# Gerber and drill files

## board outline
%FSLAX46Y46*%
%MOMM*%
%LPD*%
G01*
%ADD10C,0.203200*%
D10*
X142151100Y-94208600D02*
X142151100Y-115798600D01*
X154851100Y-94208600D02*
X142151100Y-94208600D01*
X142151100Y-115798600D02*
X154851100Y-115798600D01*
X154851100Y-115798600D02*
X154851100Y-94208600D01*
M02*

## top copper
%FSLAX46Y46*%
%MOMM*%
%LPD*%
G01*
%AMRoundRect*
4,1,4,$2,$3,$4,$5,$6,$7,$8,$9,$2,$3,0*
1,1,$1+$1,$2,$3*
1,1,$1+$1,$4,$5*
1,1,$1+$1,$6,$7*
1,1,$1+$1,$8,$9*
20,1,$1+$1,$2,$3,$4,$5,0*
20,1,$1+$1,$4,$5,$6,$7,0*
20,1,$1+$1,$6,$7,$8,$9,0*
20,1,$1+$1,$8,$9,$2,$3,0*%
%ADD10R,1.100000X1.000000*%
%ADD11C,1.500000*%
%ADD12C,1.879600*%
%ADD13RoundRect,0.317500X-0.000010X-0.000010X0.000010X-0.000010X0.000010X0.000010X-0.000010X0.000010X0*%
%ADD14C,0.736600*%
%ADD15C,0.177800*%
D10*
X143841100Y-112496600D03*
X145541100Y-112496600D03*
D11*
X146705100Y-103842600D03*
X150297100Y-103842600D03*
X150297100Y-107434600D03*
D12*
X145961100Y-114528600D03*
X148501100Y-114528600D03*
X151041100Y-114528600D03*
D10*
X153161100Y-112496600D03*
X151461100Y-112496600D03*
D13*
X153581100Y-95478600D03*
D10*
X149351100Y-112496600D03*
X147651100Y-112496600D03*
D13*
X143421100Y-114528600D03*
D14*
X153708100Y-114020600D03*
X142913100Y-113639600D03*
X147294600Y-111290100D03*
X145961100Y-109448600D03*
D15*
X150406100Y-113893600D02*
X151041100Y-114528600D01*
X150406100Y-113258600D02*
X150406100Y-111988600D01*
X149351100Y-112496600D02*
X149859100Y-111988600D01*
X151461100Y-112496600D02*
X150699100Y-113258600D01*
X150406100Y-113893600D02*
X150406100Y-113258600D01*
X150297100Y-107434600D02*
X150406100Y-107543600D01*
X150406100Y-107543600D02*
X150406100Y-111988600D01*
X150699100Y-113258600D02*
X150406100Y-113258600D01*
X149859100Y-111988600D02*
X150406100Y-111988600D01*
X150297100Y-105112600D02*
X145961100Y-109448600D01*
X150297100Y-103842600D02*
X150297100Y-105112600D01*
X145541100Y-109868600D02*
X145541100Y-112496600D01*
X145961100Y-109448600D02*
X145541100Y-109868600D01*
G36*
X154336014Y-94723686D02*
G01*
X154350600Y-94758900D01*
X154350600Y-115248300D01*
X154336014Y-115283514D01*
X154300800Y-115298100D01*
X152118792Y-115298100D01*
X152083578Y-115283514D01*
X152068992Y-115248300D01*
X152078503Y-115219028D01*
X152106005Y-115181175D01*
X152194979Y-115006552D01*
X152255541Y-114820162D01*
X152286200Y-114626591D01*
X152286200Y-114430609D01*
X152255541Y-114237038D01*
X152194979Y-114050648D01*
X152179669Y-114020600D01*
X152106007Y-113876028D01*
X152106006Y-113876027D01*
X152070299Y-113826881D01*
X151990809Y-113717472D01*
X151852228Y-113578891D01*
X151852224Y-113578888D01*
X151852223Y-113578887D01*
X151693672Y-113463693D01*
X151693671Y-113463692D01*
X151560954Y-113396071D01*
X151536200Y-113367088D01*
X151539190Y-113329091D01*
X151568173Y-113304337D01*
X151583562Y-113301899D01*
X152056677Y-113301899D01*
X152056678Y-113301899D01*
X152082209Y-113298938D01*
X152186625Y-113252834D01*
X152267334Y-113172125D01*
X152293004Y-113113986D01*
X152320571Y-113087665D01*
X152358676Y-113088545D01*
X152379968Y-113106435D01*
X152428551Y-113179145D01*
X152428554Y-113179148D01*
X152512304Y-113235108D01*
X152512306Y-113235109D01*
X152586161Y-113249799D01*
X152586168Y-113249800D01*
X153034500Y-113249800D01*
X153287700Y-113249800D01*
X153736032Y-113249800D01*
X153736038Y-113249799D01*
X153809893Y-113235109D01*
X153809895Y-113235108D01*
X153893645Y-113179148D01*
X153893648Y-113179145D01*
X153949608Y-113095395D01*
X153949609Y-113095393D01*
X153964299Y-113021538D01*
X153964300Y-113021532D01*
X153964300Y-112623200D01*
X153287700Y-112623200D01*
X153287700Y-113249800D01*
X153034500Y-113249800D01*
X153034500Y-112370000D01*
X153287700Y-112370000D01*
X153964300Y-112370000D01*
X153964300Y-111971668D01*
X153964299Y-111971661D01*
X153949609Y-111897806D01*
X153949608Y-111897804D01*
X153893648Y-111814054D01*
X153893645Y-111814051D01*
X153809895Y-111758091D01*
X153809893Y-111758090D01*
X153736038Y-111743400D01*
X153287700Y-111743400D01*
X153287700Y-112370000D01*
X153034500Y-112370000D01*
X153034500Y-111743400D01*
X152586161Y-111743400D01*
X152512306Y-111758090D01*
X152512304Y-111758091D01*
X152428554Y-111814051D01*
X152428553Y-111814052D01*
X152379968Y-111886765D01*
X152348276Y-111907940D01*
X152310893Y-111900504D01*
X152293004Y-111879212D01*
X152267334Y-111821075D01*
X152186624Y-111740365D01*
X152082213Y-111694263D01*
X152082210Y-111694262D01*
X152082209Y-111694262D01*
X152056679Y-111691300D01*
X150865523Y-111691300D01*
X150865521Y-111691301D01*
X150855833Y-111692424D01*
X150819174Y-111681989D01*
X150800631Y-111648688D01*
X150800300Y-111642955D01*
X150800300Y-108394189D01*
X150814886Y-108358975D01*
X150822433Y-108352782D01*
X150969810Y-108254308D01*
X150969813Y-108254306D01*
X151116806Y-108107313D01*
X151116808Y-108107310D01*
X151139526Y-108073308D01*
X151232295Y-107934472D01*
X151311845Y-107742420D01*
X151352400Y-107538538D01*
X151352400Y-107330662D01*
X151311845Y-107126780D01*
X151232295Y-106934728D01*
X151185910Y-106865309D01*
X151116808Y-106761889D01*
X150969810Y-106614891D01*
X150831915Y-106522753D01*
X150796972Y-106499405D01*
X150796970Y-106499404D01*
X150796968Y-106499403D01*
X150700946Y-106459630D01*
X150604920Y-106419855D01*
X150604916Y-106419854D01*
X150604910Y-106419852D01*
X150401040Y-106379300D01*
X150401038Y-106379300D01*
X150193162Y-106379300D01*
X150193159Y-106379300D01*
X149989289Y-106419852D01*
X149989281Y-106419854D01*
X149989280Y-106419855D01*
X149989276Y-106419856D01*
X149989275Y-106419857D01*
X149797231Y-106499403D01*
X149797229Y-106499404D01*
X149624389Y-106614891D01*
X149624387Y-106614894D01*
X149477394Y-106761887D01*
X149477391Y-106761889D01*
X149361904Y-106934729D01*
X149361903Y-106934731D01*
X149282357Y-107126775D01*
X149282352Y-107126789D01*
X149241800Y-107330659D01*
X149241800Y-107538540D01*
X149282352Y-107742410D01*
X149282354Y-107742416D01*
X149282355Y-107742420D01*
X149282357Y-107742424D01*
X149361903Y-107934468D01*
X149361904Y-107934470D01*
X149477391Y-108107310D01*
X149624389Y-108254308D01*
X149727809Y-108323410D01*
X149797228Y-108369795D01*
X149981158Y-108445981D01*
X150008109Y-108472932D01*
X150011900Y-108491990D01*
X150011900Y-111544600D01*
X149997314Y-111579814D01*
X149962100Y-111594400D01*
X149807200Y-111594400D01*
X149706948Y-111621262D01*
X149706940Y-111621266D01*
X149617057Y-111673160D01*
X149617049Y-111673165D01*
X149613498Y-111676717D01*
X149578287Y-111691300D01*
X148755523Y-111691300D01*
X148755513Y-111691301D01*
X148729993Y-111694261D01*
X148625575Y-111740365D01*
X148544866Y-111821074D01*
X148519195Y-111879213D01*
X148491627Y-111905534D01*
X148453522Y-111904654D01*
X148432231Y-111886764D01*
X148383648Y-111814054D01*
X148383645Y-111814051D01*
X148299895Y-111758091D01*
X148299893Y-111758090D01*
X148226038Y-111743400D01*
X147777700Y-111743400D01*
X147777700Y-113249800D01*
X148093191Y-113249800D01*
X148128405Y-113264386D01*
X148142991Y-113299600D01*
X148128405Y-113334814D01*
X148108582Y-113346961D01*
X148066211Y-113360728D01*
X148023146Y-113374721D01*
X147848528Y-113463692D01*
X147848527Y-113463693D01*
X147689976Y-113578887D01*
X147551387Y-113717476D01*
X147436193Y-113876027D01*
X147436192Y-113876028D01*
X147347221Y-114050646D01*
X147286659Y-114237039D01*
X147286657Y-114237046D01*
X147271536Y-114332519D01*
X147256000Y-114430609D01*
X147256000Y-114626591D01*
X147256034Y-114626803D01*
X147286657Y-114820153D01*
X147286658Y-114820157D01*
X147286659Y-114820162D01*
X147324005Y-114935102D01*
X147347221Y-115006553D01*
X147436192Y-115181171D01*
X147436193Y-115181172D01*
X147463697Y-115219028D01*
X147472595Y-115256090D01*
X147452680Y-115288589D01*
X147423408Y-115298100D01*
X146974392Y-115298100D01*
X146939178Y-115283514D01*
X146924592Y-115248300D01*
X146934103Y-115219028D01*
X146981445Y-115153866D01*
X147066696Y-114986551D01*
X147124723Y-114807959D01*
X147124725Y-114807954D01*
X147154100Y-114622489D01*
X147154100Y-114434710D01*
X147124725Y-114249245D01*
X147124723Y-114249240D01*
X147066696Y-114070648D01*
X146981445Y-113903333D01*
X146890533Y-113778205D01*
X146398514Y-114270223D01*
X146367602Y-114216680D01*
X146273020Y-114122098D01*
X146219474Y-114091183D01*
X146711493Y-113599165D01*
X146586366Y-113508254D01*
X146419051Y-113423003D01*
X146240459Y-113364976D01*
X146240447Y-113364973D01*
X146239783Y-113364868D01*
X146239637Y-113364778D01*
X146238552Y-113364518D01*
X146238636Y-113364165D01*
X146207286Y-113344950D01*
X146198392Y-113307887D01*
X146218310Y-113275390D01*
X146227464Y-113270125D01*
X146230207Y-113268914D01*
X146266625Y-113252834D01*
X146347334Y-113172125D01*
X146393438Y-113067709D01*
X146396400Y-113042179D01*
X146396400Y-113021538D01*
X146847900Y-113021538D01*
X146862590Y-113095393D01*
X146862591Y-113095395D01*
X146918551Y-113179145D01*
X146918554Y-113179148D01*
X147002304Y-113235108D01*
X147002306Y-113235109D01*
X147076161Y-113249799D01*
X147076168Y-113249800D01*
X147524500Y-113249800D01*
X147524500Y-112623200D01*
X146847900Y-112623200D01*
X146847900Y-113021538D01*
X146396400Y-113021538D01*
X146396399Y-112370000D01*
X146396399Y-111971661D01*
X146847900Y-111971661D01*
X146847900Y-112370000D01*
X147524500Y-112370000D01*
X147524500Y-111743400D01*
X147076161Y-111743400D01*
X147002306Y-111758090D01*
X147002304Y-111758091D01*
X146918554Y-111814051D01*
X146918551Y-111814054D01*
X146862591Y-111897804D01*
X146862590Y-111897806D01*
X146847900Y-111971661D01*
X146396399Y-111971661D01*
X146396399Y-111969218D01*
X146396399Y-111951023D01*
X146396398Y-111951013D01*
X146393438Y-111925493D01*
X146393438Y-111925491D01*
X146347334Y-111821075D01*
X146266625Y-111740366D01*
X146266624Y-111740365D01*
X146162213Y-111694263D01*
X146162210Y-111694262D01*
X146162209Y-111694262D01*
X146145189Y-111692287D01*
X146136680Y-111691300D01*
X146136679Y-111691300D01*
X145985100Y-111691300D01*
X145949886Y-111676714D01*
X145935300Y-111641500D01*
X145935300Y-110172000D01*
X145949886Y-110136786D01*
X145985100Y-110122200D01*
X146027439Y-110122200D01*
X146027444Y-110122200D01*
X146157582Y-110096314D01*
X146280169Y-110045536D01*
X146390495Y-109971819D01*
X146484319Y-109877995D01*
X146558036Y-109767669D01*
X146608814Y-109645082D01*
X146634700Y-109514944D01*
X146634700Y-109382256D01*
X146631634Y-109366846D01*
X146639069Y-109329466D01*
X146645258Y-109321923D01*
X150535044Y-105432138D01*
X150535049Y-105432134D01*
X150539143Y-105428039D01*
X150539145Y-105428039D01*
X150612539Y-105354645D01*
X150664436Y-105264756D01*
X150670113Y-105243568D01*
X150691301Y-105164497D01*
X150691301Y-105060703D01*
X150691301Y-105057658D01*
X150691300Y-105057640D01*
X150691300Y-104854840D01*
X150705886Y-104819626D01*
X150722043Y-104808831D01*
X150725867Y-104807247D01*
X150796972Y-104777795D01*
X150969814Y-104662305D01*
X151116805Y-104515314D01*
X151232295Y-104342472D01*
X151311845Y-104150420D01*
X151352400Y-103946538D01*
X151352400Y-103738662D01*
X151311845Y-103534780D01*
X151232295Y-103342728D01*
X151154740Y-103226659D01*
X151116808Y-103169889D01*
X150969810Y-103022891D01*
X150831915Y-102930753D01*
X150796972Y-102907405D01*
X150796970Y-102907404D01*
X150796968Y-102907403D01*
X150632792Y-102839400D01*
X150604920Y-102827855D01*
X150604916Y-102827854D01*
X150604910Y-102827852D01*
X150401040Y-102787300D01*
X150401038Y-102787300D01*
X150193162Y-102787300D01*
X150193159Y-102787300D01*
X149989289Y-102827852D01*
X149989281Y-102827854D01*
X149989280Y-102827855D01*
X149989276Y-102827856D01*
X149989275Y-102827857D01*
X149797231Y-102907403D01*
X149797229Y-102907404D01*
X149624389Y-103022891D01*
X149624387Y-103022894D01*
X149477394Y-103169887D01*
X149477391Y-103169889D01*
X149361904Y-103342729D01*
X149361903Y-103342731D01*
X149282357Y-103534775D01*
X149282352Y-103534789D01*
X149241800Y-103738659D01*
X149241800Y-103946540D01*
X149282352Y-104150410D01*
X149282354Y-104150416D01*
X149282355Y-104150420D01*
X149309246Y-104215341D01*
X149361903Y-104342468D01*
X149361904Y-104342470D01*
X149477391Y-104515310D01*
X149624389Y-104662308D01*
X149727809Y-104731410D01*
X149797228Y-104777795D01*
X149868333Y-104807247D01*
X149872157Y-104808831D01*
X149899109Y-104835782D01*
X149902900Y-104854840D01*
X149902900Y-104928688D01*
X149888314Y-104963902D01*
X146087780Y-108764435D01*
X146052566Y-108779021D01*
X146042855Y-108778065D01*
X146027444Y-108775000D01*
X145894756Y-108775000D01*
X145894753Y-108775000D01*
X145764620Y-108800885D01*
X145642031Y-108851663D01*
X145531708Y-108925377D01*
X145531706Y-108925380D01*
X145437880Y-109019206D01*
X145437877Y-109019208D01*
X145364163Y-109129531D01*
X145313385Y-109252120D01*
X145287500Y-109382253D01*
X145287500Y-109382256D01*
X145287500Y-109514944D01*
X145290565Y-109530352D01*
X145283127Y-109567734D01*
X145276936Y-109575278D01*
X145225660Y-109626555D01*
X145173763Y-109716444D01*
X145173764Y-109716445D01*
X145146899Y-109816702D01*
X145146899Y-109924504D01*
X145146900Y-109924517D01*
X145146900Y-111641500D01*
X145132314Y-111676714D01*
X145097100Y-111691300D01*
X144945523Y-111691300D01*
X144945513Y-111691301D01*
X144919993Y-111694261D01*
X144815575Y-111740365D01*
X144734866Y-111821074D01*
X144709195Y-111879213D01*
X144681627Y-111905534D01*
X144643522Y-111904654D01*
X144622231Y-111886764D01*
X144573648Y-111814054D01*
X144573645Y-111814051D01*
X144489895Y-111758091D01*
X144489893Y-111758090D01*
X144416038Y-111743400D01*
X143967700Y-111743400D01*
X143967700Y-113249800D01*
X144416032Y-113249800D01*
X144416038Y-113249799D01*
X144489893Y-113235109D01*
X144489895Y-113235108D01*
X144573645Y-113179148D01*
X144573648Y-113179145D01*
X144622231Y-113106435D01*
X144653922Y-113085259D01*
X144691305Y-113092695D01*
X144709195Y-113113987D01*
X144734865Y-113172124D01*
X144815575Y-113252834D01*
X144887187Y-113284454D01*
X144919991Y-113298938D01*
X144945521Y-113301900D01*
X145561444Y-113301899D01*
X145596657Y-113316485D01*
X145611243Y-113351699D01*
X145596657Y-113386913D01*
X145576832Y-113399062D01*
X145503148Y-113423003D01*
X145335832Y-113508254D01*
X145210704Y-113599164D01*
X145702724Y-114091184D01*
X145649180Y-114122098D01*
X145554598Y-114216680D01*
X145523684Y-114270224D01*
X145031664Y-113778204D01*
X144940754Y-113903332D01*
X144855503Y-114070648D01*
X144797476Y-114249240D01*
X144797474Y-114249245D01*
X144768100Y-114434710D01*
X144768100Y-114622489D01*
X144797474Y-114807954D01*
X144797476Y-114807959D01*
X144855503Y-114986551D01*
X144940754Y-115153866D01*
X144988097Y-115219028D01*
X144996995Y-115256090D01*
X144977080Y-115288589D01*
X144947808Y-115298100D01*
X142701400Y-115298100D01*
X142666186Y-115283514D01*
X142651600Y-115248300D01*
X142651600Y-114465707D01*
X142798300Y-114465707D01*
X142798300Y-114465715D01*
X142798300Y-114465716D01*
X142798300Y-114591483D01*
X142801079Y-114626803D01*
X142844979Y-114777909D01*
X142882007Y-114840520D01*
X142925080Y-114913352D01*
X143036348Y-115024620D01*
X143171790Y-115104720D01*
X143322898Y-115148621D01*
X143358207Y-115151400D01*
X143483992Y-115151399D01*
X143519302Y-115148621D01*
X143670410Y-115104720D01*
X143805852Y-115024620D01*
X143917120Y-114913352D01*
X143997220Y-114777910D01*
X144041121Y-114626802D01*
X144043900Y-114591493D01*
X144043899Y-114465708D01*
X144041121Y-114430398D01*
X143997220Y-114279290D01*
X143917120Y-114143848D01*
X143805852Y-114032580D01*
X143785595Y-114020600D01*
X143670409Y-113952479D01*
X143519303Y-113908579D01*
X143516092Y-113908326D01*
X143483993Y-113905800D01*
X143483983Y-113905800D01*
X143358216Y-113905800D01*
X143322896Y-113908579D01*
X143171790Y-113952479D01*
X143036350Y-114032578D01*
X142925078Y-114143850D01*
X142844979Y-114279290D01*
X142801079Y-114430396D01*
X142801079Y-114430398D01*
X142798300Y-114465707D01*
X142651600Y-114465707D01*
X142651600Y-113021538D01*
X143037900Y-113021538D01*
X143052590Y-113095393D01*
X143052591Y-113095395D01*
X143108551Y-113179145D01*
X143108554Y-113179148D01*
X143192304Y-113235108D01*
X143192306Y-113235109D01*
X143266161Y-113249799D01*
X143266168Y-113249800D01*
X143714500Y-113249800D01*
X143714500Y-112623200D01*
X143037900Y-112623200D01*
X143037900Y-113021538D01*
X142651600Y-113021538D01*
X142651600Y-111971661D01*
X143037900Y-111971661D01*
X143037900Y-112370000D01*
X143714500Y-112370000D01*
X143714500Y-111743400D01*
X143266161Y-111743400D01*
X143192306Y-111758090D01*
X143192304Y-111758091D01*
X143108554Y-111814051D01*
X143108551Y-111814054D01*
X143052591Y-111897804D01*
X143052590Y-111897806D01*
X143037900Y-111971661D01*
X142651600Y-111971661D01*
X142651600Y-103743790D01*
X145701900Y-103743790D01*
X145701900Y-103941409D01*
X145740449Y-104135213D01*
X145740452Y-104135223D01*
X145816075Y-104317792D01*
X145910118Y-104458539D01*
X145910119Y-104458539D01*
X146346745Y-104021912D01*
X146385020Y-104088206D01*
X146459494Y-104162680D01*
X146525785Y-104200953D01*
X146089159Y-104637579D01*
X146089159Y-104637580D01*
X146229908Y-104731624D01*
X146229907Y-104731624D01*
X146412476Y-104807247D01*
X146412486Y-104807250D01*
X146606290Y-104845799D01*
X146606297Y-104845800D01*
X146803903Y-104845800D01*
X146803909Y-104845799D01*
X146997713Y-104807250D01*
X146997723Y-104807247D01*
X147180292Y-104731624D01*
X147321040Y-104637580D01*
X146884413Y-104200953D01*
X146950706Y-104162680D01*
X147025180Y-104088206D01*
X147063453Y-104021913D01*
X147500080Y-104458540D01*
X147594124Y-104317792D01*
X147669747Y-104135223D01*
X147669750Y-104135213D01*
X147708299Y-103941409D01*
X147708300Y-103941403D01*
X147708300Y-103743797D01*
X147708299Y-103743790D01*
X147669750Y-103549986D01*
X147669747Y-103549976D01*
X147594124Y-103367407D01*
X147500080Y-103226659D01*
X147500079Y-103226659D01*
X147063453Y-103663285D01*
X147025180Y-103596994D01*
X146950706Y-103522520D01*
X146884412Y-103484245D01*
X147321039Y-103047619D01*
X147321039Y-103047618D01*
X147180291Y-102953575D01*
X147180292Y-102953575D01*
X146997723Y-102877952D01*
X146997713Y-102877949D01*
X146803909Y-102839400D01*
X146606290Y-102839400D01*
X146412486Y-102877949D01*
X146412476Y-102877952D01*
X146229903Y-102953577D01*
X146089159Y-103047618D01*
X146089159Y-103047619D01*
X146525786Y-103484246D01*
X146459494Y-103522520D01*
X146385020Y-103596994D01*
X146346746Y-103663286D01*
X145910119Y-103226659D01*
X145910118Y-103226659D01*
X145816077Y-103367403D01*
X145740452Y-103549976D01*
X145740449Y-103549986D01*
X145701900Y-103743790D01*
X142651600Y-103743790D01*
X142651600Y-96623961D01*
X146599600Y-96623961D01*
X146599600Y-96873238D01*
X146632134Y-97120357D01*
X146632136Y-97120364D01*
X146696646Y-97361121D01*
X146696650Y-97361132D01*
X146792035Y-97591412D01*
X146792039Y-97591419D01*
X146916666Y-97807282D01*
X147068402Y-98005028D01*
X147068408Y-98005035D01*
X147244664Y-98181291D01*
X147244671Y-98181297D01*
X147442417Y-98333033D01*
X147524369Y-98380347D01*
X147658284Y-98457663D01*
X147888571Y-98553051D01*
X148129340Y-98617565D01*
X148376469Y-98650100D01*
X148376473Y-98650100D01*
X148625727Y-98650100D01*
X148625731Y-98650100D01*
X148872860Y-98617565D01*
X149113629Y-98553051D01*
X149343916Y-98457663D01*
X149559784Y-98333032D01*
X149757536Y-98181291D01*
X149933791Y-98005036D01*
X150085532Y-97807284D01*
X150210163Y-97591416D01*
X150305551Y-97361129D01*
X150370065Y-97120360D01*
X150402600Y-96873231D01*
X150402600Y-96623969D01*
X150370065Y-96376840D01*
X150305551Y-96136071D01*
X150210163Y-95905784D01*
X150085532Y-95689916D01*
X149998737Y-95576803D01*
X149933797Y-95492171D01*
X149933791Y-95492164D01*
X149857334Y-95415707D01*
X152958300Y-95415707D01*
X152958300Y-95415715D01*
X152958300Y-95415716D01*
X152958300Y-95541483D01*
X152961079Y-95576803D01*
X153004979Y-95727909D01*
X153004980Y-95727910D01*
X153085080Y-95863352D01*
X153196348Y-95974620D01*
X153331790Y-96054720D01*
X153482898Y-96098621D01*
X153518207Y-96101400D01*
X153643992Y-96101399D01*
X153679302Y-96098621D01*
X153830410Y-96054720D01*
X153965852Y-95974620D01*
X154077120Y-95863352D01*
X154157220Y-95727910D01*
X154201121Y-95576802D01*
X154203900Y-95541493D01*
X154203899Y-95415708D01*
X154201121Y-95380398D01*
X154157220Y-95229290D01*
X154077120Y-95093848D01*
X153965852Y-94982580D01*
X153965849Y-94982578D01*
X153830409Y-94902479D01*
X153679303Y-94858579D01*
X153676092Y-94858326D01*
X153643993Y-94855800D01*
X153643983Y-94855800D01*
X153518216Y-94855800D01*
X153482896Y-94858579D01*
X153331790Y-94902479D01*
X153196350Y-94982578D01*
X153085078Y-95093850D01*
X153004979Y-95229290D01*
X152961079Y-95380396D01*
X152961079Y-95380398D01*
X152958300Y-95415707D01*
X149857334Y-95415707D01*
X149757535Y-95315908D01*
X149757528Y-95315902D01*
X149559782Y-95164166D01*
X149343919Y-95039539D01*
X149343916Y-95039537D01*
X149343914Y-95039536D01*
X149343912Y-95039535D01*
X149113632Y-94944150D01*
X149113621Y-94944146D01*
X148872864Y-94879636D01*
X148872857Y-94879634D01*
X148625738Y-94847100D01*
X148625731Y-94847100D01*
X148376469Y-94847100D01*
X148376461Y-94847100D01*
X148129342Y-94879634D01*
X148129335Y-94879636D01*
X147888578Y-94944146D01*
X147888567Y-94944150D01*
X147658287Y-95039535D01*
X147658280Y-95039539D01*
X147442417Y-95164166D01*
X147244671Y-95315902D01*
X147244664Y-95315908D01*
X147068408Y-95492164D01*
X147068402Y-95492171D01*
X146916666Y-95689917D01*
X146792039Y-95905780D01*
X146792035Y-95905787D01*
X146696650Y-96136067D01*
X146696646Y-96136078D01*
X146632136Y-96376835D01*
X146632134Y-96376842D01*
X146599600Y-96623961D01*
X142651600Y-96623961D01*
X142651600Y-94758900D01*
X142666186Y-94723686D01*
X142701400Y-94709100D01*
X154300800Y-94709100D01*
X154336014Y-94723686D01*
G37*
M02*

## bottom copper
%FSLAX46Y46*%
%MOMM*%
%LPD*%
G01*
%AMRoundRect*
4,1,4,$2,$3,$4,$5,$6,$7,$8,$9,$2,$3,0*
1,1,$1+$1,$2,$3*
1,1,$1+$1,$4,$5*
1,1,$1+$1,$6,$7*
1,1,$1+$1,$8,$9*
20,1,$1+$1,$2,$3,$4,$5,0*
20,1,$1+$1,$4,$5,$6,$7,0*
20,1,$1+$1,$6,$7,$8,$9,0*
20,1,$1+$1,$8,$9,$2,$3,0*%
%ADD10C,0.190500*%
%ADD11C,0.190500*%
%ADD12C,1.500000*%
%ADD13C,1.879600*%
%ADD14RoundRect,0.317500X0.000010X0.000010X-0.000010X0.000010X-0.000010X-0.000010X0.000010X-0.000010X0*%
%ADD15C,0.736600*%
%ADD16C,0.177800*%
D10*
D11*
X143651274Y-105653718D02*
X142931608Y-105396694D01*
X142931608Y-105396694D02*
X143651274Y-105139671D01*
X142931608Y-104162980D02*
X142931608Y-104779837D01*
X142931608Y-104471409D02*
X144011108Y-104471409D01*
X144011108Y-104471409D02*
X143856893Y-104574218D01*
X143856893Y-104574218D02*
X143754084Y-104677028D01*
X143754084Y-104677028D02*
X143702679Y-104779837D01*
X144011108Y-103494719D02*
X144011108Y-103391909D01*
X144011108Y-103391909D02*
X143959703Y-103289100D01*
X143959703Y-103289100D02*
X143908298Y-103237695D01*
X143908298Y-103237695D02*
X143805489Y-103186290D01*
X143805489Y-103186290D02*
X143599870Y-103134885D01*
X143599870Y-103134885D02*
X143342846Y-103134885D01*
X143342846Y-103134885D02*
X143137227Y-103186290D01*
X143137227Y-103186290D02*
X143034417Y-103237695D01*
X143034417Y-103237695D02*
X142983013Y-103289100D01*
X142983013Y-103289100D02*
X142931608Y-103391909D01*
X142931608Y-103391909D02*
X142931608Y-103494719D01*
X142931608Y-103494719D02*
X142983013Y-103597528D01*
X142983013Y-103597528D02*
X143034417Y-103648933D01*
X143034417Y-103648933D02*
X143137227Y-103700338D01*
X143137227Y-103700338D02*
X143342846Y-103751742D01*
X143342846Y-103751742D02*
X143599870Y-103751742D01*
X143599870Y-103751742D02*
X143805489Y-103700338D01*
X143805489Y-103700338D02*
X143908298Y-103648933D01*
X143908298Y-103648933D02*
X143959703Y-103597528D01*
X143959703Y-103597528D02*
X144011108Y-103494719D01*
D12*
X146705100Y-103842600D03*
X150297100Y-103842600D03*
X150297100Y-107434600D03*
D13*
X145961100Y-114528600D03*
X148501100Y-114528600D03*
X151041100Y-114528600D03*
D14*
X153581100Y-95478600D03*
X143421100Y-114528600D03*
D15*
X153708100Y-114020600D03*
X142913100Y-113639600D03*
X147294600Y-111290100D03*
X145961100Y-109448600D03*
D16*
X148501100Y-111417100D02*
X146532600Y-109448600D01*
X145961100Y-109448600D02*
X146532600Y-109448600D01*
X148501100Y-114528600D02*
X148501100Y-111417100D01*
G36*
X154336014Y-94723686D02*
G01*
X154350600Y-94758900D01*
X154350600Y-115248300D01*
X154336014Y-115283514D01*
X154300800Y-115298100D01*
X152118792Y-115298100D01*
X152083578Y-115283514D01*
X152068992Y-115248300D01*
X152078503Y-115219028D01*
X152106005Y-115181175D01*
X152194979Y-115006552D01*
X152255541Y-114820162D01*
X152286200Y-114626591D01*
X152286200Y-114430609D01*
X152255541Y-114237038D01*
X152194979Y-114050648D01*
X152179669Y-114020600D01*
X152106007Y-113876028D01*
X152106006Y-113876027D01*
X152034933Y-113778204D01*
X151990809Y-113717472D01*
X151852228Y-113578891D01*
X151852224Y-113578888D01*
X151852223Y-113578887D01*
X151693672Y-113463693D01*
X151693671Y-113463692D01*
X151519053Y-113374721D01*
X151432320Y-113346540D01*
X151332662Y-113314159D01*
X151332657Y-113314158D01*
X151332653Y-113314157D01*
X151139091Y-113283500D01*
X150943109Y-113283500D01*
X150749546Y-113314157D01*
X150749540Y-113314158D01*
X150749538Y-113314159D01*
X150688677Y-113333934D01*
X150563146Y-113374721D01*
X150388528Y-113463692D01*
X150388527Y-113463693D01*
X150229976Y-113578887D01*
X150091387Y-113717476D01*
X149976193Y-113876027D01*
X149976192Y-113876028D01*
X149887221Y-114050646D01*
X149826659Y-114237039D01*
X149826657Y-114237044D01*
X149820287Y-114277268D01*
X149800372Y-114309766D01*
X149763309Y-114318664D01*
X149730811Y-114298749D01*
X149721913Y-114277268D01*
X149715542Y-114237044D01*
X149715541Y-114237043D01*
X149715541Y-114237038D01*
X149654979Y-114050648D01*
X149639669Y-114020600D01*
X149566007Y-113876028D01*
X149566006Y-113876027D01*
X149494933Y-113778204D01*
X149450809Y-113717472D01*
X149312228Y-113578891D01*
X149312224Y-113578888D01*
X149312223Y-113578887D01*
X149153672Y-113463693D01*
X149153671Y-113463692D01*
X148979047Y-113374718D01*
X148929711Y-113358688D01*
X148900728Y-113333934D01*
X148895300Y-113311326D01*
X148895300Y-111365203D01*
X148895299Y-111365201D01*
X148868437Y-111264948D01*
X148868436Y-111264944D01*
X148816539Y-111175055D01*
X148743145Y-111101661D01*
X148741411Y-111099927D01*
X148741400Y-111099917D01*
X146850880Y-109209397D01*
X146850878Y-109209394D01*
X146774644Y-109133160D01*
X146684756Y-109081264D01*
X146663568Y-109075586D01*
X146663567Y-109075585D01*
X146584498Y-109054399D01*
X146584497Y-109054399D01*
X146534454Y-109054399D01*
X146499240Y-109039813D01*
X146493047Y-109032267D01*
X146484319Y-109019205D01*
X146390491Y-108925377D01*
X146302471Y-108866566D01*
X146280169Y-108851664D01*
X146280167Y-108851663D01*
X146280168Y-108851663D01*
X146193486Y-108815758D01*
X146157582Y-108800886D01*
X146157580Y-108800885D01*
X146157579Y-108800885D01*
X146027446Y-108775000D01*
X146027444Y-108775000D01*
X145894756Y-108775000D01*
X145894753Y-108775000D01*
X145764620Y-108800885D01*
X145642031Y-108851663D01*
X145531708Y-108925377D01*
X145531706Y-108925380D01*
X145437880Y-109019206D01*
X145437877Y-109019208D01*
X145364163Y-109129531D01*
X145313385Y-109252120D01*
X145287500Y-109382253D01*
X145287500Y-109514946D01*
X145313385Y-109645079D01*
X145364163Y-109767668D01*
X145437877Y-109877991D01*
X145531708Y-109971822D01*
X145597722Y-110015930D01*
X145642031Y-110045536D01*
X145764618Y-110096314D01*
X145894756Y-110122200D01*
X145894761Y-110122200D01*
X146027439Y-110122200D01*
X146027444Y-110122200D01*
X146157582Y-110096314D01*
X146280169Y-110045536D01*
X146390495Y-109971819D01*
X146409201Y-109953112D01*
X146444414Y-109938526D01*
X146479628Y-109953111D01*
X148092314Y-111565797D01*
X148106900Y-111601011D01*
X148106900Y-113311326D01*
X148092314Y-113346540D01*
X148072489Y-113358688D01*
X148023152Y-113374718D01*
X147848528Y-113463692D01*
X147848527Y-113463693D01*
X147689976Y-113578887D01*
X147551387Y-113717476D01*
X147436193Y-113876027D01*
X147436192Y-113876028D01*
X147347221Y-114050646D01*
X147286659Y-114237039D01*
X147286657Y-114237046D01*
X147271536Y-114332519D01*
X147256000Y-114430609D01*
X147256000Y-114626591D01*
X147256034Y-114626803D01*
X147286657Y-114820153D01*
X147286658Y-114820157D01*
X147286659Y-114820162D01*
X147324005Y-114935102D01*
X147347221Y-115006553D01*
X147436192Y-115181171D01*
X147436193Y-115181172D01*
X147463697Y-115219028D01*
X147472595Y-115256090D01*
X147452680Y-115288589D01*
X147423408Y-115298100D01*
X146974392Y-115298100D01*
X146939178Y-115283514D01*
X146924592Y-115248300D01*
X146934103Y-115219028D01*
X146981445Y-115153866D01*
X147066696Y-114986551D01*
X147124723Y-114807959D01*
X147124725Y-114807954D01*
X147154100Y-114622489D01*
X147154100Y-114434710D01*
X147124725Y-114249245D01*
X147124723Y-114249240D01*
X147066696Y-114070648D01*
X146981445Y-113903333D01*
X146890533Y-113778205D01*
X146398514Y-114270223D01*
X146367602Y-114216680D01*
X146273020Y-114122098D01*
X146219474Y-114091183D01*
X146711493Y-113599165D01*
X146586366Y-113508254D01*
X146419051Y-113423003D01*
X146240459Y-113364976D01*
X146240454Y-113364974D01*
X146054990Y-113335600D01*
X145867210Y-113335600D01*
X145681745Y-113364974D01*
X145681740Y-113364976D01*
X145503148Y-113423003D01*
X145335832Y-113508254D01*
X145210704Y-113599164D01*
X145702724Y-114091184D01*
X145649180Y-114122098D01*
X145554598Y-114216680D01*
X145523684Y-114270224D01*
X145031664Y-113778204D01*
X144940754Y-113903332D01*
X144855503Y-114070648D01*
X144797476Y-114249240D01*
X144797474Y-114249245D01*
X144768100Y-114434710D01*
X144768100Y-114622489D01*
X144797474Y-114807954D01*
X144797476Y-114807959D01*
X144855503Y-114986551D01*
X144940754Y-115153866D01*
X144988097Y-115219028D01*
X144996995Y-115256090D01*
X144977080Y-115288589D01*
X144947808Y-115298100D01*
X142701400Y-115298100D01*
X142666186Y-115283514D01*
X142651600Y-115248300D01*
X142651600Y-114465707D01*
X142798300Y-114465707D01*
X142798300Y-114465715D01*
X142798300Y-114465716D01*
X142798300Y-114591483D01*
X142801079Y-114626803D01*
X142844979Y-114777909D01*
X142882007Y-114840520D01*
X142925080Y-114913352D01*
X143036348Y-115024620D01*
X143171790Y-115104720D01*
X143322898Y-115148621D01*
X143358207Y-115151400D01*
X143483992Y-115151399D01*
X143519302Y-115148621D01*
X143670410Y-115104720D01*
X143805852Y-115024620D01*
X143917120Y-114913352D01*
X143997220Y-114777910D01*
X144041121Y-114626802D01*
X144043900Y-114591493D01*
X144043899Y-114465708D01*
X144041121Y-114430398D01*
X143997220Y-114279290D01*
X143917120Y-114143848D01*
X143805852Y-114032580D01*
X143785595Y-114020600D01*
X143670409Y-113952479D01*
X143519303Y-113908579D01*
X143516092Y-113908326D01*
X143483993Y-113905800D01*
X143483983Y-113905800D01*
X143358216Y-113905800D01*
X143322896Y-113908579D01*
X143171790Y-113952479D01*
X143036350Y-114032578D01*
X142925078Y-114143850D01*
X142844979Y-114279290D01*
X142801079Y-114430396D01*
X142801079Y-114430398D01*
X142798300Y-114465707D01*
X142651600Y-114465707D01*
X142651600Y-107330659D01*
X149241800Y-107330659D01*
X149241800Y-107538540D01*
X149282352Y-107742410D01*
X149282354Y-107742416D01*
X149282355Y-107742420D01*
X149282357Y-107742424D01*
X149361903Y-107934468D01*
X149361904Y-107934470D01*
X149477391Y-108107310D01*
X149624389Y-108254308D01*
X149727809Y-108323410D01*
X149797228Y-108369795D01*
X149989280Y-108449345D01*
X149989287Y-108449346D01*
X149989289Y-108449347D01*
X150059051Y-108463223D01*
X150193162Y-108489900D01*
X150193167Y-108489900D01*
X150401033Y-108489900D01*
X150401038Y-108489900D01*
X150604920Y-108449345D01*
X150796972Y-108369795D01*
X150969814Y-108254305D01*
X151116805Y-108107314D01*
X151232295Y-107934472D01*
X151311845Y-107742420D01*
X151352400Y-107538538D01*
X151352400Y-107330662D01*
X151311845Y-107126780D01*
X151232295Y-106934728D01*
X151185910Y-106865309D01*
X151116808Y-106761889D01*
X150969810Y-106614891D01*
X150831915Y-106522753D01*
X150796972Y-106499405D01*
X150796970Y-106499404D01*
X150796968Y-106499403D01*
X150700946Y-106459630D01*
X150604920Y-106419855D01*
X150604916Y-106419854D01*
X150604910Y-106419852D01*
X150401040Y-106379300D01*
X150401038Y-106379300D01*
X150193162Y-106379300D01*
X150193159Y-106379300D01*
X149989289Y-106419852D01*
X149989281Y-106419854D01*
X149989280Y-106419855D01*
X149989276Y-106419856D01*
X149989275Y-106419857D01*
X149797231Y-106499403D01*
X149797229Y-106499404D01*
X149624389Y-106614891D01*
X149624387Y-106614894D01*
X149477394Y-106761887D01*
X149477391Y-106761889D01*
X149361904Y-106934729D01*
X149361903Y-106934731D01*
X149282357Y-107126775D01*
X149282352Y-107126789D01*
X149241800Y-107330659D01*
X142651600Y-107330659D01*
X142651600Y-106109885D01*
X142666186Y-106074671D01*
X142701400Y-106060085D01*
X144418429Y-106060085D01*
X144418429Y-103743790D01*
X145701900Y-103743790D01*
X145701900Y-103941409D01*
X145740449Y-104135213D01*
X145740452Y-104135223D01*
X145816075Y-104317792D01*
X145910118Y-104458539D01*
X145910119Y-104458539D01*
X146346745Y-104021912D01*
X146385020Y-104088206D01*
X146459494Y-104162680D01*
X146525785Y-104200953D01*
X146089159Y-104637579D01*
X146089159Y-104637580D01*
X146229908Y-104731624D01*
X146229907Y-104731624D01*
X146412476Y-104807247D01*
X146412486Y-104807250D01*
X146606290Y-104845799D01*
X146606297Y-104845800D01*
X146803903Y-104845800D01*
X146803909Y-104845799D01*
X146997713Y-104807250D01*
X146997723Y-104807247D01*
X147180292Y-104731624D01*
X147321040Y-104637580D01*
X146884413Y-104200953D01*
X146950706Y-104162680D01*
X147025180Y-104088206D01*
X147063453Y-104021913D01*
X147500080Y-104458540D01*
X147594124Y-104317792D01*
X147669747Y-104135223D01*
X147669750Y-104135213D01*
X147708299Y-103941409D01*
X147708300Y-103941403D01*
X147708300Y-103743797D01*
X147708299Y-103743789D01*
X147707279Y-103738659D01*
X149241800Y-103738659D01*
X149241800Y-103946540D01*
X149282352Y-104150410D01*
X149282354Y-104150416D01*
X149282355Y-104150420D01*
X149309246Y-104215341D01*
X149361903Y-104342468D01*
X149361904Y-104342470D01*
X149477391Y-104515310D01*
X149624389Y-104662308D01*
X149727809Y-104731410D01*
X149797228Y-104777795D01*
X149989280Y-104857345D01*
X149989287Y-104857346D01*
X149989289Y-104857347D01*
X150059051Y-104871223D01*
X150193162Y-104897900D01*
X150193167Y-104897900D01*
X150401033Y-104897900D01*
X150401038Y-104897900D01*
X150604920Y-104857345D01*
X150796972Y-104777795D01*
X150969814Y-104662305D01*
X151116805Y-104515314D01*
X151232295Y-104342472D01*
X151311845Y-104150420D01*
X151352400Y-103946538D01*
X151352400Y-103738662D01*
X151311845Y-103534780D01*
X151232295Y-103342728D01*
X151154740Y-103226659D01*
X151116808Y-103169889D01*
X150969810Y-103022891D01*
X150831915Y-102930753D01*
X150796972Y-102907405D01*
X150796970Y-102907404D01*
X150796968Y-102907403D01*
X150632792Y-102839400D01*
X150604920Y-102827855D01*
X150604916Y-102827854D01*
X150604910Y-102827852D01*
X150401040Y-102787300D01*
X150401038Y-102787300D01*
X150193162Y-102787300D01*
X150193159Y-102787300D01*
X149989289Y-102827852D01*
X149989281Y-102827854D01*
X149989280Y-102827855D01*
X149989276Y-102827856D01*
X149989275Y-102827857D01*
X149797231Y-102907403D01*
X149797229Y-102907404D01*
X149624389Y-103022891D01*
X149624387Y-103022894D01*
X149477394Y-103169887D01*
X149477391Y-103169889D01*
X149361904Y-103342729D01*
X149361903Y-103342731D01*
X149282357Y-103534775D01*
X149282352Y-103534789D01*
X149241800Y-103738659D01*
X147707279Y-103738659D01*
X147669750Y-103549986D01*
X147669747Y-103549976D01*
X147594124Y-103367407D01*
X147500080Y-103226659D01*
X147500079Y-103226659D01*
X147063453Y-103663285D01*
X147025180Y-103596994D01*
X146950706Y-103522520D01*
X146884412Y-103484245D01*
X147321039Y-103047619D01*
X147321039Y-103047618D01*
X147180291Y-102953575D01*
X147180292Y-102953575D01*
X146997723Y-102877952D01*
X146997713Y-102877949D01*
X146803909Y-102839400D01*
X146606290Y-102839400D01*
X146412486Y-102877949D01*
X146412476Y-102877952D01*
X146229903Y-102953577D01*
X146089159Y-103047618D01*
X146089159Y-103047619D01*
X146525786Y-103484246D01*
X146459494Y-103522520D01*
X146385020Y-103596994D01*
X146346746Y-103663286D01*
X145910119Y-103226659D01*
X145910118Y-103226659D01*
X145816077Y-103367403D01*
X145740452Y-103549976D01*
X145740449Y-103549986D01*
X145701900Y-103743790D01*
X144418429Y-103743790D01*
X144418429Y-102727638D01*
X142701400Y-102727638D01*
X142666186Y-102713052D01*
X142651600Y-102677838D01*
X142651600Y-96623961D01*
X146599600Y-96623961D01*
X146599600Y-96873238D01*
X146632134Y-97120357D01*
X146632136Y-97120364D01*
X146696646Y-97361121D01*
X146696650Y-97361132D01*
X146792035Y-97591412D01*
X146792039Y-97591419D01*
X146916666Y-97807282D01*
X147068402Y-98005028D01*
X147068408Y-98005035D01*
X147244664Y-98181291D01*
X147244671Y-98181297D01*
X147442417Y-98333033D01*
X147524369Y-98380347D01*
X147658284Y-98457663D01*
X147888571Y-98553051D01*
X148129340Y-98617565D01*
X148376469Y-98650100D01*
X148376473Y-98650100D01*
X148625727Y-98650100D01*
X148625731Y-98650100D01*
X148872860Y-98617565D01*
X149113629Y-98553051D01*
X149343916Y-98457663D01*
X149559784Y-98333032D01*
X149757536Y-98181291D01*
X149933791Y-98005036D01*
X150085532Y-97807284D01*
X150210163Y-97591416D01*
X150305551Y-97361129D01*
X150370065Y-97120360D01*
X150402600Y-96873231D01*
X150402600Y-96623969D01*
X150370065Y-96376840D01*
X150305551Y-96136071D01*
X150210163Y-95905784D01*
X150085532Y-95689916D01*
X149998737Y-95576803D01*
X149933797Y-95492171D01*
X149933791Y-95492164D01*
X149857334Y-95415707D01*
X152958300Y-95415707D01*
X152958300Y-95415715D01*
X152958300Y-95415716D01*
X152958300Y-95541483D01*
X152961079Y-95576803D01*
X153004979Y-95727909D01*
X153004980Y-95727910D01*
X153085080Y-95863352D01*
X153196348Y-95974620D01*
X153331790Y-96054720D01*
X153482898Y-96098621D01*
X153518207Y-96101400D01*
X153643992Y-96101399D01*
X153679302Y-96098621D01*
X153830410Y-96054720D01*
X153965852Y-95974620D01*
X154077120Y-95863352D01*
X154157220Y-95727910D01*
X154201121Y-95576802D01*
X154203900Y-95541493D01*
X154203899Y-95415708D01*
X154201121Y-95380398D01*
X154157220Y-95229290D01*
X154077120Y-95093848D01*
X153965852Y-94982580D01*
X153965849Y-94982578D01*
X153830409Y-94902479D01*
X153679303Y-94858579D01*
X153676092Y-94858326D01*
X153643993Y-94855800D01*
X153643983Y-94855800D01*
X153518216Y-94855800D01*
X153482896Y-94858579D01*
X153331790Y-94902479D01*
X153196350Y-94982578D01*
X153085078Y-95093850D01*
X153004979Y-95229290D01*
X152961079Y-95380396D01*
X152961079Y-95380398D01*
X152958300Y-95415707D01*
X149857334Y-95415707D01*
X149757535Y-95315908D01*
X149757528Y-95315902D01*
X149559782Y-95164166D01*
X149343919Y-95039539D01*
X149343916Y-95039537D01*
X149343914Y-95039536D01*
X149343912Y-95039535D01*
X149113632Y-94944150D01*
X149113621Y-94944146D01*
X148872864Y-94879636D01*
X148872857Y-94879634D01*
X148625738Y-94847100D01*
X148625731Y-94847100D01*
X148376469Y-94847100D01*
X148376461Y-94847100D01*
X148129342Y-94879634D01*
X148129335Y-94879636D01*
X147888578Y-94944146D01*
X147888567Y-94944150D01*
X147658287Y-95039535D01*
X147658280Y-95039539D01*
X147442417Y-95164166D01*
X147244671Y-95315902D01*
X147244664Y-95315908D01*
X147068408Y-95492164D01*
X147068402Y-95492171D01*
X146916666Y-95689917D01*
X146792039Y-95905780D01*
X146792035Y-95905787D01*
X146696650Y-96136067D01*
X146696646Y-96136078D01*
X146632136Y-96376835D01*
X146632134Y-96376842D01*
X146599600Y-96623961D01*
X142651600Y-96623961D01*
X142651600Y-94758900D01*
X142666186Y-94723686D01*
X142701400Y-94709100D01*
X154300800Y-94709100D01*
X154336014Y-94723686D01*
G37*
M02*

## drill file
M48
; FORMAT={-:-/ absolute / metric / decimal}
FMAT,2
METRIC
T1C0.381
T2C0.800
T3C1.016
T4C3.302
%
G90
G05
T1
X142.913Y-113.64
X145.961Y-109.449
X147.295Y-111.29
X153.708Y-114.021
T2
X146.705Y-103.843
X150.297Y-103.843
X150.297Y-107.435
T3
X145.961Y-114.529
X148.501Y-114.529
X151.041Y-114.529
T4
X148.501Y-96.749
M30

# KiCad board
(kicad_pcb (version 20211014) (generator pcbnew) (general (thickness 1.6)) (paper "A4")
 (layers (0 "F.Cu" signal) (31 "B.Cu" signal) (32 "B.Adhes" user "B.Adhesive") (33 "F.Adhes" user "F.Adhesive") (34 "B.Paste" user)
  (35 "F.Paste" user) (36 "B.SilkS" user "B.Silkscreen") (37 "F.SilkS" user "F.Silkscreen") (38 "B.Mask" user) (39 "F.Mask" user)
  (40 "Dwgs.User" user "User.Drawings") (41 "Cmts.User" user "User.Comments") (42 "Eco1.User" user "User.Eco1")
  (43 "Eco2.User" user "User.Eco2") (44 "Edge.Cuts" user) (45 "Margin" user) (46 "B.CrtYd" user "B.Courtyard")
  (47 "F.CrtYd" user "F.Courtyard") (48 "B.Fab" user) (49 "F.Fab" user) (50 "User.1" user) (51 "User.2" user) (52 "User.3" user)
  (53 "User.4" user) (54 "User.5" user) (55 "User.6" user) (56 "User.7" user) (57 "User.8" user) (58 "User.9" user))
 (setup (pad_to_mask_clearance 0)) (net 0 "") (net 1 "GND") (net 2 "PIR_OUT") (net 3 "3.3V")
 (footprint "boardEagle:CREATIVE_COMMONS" (layer "F.Cu") (at 123.1011 124.6886)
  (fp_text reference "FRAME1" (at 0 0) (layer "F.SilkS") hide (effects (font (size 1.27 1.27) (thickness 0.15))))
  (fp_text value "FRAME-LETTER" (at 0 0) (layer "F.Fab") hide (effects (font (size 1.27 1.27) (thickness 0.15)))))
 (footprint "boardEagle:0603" (layer "F.Cu") (at 144.6911 112.4966)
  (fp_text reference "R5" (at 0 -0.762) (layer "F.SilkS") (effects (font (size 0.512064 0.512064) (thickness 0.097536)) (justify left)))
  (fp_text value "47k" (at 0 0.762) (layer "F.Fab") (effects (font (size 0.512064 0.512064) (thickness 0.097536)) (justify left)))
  (pad "1" smd rect (at -0.85 0) (size 1.1 1) (layers "F.Cu" "F.Paste" "F.Mask") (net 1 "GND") (solder_mask_margin 0.1016))
  (pad "2" smd rect (at 0.85 0) (size 1.1 1) (layers "F.Cu" "F.Paste" "F.Mask") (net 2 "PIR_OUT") (solder_mask_margin 0.1016)))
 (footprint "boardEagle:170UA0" (layer "F.Cu") (at 143.4211 99.9236 90)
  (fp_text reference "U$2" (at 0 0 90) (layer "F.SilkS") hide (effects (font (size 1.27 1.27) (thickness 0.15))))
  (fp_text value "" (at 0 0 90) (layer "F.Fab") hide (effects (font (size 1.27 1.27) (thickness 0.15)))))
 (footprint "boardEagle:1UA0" (layer "F.Cu") (at 153.5811 99.9236 90)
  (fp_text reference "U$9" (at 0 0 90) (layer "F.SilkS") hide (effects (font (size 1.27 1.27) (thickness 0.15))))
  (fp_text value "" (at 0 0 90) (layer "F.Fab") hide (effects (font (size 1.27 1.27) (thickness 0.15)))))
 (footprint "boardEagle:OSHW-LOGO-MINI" (layer "F.Cu") (at 153.3906 110.7186)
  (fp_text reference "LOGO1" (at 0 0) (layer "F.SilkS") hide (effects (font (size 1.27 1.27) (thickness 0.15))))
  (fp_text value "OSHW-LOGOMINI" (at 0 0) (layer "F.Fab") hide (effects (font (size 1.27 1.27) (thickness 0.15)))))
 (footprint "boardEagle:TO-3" (layer "F.Cu") (at 148.5011 105.6386)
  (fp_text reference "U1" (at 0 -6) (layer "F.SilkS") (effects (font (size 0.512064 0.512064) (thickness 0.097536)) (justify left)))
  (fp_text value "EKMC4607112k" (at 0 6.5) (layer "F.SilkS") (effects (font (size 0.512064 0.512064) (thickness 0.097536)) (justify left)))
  (pad "GND" thru_hole circle (at -1.796 -1.796) (size 1.5 1.5) (drill 0.8) (layers *.Cu) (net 1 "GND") (solder_mask_margin 0.1016))
  (pad "OUT" thru_hole circle (at 1.796 -1.796) (size 1.5 1.5) (drill 0.8) (layers *.Cu) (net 2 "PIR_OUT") (solder_mask_margin 0.1016))
  (pad "VDD" thru_hole circle (at 1.796 1.796) (size 1.5 1.5) (drill 0.8) (layers *.Cu) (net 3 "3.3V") (solder_mask_margin 0.1016)))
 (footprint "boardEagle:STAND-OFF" (layer "F.Cu") (at 148.5011 96.7486)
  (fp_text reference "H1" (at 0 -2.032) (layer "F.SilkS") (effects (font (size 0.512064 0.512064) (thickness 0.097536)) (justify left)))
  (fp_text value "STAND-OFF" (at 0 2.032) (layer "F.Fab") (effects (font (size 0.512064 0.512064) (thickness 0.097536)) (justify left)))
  (pad "" np_thru_hole circle (at 0 0) (size 3.302 3.302) (drill 3.302) (layers *.Cu *.Mask)))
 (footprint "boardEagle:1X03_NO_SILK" (layer "F.Cu") (at 145.9611 114.5286)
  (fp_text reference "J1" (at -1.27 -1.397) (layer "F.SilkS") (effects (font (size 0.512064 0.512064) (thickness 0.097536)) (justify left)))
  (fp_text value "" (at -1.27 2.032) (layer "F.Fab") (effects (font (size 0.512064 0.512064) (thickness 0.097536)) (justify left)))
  (pad "1" thru_hole circle (at 0 0 90) (size 1.8796 1.8796) (drill 1.016) (layers *.Cu *.Mask) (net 1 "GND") (solder_mask_margin 0.1016))
  (pad "2" thru_hole circle (at 2.54 0 90) (size 1.8796 1.8796) (drill 1.016) (layers *.Cu *.Mask) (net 2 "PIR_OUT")
   (solder_mask_margin 0.1016))
  (pad "3" thru_hole circle (at 5.08 0 90) (size 1.8796 1.8796) (drill 1.016) (layers *.Cu *.Mask) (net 3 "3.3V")
   (solder_mask_margin 0.1016)))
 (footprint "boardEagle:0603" (layer "F.Cu") (at 152.3111 112.4966 180)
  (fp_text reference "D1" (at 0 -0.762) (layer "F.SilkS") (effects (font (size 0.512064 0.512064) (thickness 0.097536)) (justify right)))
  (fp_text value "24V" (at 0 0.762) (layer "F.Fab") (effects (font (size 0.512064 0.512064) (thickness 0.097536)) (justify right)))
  (pad "1" smd rect (at -0.85 0 180) (size 1.1 1) (layers "F.Cu" "F.Paste" "F.Mask") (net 1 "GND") (solder_mask_margin 0.1016))
  (pad "2" smd rect (at 0.85 0 180) (size 1.1 1) (layers "F.Cu" "F.Paste" "F.Mask") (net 3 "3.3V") (solder_mask_margin 0.1016)))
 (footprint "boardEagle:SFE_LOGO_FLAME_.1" (layer "F.Cu") (at 143.6116 110.5916)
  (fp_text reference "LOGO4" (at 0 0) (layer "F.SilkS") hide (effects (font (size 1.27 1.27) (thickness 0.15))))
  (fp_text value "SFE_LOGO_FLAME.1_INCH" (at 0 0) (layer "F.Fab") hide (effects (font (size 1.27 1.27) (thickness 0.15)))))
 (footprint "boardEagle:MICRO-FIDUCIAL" (layer "F.Cu") (at 153.5811 95.4786)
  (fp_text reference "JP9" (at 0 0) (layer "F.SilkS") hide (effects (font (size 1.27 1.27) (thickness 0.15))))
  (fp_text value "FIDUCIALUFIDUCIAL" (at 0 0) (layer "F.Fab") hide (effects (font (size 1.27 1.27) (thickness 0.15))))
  (pad "1" smd roundrect (at 0 0) (size 0.635 0.635) (layers "F.Cu" "F.Mask") (roundrect_rratio 0.5) (solder_mask_margin 0.1016)))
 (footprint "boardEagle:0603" (layer "F.Cu") (at 148.5011 112.4966 180)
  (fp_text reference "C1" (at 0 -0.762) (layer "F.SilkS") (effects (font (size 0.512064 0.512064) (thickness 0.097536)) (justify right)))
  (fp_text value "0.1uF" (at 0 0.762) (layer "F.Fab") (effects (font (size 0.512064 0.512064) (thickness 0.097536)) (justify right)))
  (pad "1" smd rect (at -0.85 0 180) (size 1.1 1) (layers "F.Cu" "F.Paste" "F.Mask") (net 3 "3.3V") (solder_mask_margin 0.1016))
  (pad "2" smd rect (at 0.85 0 180) (size 1.1 1) (layers "F.Cu" "F.Paste" "F.Mask") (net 1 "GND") (solder_mask_margin 0.1016)))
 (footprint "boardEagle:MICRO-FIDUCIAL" (layer "F.Cu") (at 143.4211 114.5286)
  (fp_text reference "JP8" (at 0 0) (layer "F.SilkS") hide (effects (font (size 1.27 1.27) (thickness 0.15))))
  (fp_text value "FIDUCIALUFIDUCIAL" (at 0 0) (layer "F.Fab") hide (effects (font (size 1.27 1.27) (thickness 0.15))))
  (pad "1" smd roundrect (at 0 0) (size 0.635 0.635) (layers "F.Cu" "F.Mask") (roundrect_rratio 0.5) (solder_mask_margin 0.1016)))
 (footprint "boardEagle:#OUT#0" (layer "B.Cu") (at 148.5011 114.0841 90)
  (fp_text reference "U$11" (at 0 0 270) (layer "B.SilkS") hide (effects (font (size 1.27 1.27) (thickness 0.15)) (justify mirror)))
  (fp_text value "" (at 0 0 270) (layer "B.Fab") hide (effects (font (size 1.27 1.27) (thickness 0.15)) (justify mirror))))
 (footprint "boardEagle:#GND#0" (layer "B.Cu") (at 145.9611 114.0206 90)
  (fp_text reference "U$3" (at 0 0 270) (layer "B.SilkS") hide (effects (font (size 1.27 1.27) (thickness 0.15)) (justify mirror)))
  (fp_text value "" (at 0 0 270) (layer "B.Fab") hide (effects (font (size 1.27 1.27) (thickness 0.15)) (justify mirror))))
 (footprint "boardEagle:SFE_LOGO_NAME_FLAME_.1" (layer "B.Cu") (at 148.5011 101.8286 180)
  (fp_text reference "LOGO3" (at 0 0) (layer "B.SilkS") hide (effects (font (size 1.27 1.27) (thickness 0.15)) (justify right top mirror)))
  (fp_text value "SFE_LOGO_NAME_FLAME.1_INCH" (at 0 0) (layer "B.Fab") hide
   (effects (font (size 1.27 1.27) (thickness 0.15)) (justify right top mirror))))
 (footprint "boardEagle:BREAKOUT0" (layer "B.Cu") (at 152.6286 106.0196 180)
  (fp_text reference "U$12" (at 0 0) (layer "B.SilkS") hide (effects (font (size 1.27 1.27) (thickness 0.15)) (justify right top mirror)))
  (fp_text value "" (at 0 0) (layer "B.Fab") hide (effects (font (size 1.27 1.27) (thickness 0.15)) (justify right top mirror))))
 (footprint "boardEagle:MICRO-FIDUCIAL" (layer "B.Cu") (at 153.5811 95.4786 180)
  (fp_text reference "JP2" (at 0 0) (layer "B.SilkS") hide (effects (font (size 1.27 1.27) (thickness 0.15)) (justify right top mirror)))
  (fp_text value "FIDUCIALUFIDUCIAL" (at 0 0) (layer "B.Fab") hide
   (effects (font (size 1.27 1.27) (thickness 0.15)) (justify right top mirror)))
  (pad "1" smd roundrect (at 0 0 180) (size 0.635 0.635) (layers "B.Cu" "B.Mask") (roundrect_rratio 0.5) (solder_mask_margin 0.1016)))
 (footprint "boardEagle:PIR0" (layer "B.Cu") (at 150.2156 104.8131 180)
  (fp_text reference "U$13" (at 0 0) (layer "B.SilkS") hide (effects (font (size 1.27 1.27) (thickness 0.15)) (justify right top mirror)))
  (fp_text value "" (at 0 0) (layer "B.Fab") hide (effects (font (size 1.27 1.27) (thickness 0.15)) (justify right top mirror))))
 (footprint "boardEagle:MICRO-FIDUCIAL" (layer "B.Cu") (at 143.4211 114.5286 180)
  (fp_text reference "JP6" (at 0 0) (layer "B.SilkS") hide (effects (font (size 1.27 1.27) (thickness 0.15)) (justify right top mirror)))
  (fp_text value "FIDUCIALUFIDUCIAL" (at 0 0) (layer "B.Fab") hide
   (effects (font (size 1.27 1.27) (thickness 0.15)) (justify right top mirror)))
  (pad "1" smd roundrect (at 0 0 180) (size 0.635 0.635) (layers "B.Cu" "B.Mask") (roundrect_rratio 0.5) (solder_mask_margin 0.1016)))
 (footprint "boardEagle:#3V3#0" (layer "B.Cu") (at 151.0411 114.0206 90)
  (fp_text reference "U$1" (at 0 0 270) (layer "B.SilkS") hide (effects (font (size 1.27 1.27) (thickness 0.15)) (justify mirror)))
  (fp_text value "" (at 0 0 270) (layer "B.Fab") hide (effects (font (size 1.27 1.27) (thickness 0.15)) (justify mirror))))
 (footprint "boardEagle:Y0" (layer "B.Cu") (at 153.5811 106.9086 180)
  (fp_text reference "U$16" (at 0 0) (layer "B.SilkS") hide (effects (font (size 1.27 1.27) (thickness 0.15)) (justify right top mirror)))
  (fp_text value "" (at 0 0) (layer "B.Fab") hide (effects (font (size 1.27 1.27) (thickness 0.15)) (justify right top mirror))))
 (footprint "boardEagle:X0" (layer "B.Cu") (at 154.3431 105.7656 180)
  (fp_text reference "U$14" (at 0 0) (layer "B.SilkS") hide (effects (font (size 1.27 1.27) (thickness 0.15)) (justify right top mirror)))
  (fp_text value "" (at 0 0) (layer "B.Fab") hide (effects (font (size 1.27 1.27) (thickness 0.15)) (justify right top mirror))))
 (gr_line (start 142.1511 94.2086) (end 142.1511 115.7986) (layer "Edge.Cuts") (width 0.2032))
 (gr_line (start 154.8511 94.2086) (end 142.1511 94.2086) (layer "Edge.Cuts") (width 0.2032))
 (gr_line (start 142.1511 115.7986) (end 154.8511 115.7986) (layer "Edge.Cuts") (width 0.2032))
 (gr_line (start 154.8511 115.7986) (end 154.8511 94.2086) (layer "Edge.Cuts") (width 0.2032))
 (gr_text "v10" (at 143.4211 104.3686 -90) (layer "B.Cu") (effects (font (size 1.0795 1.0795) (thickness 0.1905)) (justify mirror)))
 (via (at 153.7081 114.0206) (size 0.7366) (drill 0.381) (layers "F.Cu" "B.Cu") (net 1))
 (via (at 142.9131 113.6396) (size 0.7366) (drill 0.381) (layers "F.Cu" "B.Cu") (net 1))
 (via (at 147.2946 111.2901) (size 0.7366) (drill 0.381) (layers "F.Cu" "B.Cu") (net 1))
 (segment (start 150.4061 113.8936) (end 151.0411 114.5286) (width 0.1778) (layer "F.Cu") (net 3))
 (segment (start 150.4061 113.2586) (end 150.4061 111.9886) (width 0.1778) (layer "F.Cu") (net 3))
 (segment (start 149.3511 112.4966) (end 149.8591 111.9886) (width 0.1778) (layer "F.Cu") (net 3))
 (segment (start 151.4611 112.4966) (end 150.6991 113.2586) (width 0.1778) (layer "F.Cu") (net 3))
 (segment (start 150.4061 113.8936) (end 150.4061 113.2586) (width 0.1778) (layer "F.Cu") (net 3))
 (segment (start 150.2971 107.4346) (end 150.4061 107.5436) (width 0.1778) (layer "F.Cu") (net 3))
 (segment (start 150.4061 107.5436) (end 150.4061 111.9886) (width 0.1778) (layer "F.Cu") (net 3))
 (segment (start 150.6991 113.2586) (end 150.4061 113.2586) (width 0.1778) (layer "F.Cu") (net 3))
 (segment (start 149.8591 111.9886) (end 150.4061 111.9886) (width 0.1778) (layer "F.Cu") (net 3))
 (segment (start 150.2971 105.1126) (end 145.9611 109.4486) (width 0.1778) (layer "F.Cu") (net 2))
 (segment (start 150.2971 103.8426) (end 150.2971 105.1126) (width 0.1778) (layer "F.Cu") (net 2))
 (segment (start 145.5411 109.8686) (end 145.5411 112.4966) (width 0.1778) (layer "F.Cu") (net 2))
 (segment (start 145.9611 109.4486) (end 145.5411 109.8686) (width 0.1778) (layer "F.Cu") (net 2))
 (via (at 145.9611 109.4486) (size 0.7366) (drill 0.381) (layers "F.Cu" "B.Cu") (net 2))
 (segment (start 148.5011 111.4171) (end 146.5326 109.4486) (width 0.1778) (layer "B.Cu") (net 2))
 (segment (start 145.9611 109.4486) (end 146.5326 109.4486) (width 0.1778) (layer "B.Cu") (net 2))
 (segment (start 148.5011 114.5286) (end 148.5011 111.4171) (width 0.1778) (layer "B.Cu") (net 2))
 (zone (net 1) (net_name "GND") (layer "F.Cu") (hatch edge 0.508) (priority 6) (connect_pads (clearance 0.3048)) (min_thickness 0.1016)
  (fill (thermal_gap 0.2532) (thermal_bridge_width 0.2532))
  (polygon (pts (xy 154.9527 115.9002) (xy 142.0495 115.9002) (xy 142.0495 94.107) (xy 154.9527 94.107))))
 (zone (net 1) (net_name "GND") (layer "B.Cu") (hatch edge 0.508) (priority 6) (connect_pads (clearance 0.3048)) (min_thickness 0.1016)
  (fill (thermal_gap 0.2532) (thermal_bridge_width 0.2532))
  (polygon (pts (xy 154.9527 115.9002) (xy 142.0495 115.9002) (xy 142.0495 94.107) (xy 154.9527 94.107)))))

